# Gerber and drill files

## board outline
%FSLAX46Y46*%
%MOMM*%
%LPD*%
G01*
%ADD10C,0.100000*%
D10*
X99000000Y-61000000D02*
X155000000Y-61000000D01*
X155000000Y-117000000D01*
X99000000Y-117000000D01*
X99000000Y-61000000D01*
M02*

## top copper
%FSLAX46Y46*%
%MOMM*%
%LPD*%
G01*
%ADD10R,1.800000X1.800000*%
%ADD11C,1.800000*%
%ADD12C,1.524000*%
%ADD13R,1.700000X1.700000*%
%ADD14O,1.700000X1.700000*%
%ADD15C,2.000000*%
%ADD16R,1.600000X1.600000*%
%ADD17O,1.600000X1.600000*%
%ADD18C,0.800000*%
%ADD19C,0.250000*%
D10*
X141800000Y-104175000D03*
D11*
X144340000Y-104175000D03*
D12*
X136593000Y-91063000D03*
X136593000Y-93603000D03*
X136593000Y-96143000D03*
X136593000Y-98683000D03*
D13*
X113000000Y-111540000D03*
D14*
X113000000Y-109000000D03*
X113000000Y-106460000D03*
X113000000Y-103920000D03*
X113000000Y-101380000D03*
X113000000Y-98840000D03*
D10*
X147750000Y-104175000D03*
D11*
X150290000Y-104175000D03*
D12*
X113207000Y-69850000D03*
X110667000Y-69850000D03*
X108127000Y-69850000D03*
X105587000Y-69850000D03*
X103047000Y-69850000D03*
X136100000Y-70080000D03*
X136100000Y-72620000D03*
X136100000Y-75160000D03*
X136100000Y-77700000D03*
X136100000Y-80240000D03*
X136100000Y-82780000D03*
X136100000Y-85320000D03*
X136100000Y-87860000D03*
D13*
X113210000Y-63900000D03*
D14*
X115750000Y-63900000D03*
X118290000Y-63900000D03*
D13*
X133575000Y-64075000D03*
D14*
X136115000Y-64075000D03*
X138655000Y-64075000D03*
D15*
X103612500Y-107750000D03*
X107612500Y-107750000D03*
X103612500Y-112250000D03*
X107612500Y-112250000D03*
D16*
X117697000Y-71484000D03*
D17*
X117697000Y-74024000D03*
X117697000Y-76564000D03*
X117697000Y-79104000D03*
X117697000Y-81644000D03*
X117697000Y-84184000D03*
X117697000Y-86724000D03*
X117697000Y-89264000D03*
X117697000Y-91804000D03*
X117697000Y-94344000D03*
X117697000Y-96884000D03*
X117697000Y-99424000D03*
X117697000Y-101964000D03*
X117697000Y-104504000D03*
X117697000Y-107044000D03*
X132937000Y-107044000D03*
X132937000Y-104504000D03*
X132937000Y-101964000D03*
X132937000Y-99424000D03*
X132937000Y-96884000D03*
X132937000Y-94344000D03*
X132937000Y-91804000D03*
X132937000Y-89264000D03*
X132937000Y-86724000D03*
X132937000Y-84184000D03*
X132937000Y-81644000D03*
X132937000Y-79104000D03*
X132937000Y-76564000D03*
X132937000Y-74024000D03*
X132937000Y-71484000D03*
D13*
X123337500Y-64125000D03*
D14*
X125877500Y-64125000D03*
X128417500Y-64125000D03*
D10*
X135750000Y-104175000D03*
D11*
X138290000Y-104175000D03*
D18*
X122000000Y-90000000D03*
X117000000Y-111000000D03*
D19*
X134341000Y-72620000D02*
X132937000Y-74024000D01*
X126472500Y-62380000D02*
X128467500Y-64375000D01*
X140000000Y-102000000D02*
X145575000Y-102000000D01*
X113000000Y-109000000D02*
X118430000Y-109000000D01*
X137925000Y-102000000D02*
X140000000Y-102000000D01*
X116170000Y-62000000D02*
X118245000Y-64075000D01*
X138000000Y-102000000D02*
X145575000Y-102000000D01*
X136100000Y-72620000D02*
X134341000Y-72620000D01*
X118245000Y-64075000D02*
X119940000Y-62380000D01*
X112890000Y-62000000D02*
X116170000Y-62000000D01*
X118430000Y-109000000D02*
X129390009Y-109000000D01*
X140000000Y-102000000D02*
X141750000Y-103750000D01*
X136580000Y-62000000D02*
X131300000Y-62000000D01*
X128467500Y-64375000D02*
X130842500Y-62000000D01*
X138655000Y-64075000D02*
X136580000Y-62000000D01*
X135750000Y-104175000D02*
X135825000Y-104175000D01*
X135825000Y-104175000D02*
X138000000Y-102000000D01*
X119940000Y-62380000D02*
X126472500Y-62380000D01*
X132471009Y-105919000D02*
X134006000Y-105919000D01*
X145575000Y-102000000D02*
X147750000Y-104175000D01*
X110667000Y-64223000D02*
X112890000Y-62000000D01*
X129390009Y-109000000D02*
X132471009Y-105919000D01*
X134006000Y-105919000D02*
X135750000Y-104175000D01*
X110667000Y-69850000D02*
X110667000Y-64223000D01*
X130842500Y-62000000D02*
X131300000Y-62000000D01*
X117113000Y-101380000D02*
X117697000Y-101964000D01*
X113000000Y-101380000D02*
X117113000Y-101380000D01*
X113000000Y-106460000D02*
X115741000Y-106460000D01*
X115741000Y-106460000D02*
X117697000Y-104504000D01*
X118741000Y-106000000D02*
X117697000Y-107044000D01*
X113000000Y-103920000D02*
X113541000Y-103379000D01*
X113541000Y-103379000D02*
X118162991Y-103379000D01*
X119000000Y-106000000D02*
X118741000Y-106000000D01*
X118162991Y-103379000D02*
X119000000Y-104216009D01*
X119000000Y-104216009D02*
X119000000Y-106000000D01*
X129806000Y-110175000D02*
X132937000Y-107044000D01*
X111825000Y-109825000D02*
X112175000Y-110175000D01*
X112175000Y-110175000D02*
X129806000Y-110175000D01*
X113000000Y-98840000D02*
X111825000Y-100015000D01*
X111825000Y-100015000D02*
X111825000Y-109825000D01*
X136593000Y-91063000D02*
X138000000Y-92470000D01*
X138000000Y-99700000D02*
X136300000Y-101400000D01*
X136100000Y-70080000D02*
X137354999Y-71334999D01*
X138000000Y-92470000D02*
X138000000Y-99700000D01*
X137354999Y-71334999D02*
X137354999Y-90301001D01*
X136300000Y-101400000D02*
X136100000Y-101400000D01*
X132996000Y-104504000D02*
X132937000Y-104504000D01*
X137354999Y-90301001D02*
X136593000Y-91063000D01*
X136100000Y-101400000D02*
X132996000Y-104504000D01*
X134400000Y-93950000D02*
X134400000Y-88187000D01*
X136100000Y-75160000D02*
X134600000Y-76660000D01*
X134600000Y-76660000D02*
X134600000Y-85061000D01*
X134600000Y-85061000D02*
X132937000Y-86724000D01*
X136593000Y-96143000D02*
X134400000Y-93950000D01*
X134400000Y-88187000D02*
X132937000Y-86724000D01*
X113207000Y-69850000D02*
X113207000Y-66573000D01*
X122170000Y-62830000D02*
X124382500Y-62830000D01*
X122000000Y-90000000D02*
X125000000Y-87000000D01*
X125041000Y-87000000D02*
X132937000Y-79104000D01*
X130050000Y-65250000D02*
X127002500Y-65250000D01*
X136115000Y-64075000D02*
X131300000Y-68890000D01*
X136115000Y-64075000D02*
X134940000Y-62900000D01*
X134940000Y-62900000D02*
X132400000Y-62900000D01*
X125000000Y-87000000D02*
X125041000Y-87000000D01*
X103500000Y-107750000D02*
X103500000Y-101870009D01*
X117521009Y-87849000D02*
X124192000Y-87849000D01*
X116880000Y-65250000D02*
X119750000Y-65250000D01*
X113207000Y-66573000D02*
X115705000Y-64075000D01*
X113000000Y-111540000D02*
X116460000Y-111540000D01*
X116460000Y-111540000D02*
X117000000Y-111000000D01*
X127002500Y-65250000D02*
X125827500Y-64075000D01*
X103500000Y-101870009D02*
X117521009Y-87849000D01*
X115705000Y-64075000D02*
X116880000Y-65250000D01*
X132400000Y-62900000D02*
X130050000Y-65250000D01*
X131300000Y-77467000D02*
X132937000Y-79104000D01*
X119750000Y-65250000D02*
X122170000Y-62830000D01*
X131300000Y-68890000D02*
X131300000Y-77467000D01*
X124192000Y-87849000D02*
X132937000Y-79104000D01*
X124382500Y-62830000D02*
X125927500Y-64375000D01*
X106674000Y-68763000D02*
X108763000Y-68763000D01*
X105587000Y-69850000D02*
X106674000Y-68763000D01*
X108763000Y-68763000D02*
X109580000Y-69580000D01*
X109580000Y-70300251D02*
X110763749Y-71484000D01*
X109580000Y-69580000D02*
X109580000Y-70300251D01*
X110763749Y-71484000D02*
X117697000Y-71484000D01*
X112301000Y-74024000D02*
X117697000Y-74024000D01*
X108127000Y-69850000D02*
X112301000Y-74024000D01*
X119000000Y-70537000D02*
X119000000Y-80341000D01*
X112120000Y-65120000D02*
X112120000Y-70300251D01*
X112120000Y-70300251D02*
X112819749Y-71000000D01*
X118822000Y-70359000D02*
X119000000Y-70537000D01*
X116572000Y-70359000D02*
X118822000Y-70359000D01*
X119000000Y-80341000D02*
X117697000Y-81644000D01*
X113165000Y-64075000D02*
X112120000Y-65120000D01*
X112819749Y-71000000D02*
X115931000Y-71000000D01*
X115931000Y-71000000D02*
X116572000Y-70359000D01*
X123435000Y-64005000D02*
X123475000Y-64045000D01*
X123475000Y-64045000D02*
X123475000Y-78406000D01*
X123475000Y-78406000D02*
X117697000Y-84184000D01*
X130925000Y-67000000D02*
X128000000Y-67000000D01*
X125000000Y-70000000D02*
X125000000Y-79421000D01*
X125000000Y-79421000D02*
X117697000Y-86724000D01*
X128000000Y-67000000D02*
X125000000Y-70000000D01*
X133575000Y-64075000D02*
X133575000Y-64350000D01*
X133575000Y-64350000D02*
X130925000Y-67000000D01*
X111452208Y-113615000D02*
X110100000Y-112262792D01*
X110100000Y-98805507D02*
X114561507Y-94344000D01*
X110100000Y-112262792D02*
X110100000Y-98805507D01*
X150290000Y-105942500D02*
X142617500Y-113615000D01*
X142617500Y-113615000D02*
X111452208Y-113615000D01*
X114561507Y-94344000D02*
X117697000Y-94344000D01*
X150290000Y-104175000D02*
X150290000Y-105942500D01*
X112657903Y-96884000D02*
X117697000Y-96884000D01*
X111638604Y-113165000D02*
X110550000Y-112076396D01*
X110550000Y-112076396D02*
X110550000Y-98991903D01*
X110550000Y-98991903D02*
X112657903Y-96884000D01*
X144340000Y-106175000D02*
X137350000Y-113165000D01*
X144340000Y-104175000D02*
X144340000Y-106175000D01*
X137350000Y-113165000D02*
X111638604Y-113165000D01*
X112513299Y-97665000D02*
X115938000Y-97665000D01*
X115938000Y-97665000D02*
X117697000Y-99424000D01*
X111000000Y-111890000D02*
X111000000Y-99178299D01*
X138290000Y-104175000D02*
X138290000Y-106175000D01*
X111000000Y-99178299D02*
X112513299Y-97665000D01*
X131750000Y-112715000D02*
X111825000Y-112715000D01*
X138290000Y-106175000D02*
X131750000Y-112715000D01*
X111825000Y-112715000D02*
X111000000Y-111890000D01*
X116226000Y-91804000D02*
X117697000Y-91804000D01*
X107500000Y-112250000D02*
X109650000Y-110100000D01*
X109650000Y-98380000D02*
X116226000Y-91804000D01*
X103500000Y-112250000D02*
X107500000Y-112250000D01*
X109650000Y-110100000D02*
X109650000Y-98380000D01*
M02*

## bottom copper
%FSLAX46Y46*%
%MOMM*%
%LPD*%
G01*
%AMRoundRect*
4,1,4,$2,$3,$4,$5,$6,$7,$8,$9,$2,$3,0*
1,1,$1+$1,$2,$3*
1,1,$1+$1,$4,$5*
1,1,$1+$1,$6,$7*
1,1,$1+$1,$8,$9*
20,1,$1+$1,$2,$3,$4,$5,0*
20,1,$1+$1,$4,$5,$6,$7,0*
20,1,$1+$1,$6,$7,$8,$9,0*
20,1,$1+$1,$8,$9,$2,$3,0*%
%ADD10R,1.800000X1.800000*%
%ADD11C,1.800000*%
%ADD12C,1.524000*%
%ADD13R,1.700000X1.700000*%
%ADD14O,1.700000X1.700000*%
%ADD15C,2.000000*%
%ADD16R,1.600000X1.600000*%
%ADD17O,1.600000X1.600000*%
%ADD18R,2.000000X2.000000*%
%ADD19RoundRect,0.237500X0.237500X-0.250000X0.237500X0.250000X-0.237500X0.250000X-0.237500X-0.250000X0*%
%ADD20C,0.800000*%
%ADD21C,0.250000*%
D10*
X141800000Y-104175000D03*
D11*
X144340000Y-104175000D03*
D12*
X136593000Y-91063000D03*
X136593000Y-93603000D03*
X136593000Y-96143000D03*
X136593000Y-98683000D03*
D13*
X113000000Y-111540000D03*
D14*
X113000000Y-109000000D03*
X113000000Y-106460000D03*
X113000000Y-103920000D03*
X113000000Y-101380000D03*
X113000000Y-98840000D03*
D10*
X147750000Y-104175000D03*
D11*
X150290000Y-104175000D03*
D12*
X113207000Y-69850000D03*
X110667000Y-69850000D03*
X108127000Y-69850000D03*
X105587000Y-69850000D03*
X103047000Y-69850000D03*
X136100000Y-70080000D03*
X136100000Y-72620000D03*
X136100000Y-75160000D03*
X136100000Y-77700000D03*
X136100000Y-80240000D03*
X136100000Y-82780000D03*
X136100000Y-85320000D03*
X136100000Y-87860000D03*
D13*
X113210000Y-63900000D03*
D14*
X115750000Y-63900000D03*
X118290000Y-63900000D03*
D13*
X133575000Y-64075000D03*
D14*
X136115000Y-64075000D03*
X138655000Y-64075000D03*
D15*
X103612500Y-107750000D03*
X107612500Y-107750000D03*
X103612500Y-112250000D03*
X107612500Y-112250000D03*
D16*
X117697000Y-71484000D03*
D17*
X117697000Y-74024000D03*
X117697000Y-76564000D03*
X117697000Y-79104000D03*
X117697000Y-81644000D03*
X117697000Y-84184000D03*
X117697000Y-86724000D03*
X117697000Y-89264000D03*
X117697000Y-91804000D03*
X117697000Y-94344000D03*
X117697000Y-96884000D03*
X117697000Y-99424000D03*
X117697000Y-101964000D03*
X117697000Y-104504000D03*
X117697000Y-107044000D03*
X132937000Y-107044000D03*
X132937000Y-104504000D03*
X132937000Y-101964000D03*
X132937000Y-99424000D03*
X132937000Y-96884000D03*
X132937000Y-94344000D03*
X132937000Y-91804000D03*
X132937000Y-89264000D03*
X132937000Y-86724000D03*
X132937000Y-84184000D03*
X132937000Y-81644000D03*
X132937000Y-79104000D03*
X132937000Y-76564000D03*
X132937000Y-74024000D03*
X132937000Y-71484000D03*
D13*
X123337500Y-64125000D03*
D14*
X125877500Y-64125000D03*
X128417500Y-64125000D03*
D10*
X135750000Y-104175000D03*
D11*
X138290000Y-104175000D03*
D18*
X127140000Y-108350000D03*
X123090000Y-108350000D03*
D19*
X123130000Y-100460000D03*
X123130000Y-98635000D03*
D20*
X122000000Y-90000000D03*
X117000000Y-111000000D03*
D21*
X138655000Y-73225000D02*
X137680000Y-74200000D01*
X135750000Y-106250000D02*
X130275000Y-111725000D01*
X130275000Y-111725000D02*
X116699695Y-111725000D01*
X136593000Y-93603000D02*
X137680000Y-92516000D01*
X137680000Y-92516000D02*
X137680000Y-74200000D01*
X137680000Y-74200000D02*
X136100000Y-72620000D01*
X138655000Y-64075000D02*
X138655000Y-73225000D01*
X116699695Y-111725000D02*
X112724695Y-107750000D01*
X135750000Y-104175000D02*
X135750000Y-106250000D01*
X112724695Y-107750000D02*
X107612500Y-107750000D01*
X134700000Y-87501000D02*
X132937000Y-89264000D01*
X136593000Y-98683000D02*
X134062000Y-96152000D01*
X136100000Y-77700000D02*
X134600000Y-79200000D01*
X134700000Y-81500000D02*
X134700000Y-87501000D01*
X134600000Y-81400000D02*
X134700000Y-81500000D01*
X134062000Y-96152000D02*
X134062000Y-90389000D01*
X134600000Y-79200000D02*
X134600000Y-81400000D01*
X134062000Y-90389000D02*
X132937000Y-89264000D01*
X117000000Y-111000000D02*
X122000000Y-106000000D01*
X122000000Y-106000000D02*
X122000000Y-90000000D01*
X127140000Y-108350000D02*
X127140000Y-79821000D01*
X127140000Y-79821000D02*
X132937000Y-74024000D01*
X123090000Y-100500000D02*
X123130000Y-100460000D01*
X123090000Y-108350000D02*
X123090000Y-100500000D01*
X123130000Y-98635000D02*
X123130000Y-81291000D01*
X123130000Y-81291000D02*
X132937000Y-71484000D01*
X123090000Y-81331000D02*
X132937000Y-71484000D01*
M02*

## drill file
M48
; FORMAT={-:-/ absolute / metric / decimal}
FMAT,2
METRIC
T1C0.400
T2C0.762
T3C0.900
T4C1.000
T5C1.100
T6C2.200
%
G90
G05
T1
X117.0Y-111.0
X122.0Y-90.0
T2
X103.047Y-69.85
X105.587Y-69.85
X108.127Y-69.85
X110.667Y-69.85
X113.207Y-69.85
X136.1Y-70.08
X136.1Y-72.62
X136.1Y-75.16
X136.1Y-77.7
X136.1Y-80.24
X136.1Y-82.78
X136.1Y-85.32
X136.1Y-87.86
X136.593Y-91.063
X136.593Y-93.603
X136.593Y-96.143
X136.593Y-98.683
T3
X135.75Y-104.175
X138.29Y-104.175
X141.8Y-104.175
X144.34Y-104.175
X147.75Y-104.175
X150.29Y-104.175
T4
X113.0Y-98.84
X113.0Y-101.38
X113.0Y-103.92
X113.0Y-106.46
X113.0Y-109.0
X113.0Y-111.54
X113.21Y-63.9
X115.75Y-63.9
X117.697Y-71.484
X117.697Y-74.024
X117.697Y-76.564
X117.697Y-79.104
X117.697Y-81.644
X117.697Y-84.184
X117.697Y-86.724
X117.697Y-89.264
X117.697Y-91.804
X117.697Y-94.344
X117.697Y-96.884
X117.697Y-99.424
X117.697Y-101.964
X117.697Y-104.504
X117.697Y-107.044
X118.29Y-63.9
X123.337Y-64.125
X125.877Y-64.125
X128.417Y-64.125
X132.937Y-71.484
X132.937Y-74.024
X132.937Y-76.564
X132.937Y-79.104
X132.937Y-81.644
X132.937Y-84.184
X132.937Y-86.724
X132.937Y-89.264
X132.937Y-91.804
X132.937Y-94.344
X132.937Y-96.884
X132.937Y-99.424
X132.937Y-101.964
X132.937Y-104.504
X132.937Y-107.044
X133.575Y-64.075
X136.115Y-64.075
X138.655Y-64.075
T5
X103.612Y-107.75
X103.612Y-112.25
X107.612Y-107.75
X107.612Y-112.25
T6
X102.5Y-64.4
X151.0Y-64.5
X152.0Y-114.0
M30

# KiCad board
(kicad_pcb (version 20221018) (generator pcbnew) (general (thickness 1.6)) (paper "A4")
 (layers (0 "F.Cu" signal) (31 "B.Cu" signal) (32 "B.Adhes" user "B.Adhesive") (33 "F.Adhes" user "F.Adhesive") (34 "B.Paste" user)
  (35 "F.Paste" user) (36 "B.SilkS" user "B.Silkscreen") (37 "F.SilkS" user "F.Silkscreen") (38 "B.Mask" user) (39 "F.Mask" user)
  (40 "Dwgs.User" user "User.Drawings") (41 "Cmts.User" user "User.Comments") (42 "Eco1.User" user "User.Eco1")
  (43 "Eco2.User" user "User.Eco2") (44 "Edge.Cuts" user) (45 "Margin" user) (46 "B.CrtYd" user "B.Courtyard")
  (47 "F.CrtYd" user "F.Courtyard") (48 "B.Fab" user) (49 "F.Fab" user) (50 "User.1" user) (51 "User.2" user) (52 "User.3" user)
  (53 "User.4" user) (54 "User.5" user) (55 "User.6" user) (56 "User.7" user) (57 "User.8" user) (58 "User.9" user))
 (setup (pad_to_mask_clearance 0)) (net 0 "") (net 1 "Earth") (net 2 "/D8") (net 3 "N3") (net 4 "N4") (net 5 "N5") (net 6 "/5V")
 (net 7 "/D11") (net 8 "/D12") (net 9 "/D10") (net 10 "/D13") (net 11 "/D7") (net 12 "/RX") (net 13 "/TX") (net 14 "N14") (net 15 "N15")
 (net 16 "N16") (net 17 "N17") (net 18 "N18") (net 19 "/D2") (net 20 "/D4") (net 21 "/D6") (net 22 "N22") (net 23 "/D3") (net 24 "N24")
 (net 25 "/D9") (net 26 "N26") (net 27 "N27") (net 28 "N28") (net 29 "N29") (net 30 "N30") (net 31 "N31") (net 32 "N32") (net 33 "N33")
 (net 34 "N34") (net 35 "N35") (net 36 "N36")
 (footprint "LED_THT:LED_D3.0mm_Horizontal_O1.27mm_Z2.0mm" (layer "F.Cu") (at 141.8 104.175)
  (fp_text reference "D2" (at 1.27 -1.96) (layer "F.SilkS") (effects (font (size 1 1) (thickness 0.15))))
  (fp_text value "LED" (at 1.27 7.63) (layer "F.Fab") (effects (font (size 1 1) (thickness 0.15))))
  (pad "1" thru_hole rect (at 0 0) (size 1.8 1.8) (drill 0.9) (layers "*.Cu" "*.Mask") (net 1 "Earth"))
  (pad "2" thru_hole circle (at 2.54 0) (size 1.8 1.8) (drill 0.9) (layers "*.Cu" "*.Mask") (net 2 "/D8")))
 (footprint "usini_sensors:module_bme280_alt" (layer "F.Cu") (at 136.593 98.683)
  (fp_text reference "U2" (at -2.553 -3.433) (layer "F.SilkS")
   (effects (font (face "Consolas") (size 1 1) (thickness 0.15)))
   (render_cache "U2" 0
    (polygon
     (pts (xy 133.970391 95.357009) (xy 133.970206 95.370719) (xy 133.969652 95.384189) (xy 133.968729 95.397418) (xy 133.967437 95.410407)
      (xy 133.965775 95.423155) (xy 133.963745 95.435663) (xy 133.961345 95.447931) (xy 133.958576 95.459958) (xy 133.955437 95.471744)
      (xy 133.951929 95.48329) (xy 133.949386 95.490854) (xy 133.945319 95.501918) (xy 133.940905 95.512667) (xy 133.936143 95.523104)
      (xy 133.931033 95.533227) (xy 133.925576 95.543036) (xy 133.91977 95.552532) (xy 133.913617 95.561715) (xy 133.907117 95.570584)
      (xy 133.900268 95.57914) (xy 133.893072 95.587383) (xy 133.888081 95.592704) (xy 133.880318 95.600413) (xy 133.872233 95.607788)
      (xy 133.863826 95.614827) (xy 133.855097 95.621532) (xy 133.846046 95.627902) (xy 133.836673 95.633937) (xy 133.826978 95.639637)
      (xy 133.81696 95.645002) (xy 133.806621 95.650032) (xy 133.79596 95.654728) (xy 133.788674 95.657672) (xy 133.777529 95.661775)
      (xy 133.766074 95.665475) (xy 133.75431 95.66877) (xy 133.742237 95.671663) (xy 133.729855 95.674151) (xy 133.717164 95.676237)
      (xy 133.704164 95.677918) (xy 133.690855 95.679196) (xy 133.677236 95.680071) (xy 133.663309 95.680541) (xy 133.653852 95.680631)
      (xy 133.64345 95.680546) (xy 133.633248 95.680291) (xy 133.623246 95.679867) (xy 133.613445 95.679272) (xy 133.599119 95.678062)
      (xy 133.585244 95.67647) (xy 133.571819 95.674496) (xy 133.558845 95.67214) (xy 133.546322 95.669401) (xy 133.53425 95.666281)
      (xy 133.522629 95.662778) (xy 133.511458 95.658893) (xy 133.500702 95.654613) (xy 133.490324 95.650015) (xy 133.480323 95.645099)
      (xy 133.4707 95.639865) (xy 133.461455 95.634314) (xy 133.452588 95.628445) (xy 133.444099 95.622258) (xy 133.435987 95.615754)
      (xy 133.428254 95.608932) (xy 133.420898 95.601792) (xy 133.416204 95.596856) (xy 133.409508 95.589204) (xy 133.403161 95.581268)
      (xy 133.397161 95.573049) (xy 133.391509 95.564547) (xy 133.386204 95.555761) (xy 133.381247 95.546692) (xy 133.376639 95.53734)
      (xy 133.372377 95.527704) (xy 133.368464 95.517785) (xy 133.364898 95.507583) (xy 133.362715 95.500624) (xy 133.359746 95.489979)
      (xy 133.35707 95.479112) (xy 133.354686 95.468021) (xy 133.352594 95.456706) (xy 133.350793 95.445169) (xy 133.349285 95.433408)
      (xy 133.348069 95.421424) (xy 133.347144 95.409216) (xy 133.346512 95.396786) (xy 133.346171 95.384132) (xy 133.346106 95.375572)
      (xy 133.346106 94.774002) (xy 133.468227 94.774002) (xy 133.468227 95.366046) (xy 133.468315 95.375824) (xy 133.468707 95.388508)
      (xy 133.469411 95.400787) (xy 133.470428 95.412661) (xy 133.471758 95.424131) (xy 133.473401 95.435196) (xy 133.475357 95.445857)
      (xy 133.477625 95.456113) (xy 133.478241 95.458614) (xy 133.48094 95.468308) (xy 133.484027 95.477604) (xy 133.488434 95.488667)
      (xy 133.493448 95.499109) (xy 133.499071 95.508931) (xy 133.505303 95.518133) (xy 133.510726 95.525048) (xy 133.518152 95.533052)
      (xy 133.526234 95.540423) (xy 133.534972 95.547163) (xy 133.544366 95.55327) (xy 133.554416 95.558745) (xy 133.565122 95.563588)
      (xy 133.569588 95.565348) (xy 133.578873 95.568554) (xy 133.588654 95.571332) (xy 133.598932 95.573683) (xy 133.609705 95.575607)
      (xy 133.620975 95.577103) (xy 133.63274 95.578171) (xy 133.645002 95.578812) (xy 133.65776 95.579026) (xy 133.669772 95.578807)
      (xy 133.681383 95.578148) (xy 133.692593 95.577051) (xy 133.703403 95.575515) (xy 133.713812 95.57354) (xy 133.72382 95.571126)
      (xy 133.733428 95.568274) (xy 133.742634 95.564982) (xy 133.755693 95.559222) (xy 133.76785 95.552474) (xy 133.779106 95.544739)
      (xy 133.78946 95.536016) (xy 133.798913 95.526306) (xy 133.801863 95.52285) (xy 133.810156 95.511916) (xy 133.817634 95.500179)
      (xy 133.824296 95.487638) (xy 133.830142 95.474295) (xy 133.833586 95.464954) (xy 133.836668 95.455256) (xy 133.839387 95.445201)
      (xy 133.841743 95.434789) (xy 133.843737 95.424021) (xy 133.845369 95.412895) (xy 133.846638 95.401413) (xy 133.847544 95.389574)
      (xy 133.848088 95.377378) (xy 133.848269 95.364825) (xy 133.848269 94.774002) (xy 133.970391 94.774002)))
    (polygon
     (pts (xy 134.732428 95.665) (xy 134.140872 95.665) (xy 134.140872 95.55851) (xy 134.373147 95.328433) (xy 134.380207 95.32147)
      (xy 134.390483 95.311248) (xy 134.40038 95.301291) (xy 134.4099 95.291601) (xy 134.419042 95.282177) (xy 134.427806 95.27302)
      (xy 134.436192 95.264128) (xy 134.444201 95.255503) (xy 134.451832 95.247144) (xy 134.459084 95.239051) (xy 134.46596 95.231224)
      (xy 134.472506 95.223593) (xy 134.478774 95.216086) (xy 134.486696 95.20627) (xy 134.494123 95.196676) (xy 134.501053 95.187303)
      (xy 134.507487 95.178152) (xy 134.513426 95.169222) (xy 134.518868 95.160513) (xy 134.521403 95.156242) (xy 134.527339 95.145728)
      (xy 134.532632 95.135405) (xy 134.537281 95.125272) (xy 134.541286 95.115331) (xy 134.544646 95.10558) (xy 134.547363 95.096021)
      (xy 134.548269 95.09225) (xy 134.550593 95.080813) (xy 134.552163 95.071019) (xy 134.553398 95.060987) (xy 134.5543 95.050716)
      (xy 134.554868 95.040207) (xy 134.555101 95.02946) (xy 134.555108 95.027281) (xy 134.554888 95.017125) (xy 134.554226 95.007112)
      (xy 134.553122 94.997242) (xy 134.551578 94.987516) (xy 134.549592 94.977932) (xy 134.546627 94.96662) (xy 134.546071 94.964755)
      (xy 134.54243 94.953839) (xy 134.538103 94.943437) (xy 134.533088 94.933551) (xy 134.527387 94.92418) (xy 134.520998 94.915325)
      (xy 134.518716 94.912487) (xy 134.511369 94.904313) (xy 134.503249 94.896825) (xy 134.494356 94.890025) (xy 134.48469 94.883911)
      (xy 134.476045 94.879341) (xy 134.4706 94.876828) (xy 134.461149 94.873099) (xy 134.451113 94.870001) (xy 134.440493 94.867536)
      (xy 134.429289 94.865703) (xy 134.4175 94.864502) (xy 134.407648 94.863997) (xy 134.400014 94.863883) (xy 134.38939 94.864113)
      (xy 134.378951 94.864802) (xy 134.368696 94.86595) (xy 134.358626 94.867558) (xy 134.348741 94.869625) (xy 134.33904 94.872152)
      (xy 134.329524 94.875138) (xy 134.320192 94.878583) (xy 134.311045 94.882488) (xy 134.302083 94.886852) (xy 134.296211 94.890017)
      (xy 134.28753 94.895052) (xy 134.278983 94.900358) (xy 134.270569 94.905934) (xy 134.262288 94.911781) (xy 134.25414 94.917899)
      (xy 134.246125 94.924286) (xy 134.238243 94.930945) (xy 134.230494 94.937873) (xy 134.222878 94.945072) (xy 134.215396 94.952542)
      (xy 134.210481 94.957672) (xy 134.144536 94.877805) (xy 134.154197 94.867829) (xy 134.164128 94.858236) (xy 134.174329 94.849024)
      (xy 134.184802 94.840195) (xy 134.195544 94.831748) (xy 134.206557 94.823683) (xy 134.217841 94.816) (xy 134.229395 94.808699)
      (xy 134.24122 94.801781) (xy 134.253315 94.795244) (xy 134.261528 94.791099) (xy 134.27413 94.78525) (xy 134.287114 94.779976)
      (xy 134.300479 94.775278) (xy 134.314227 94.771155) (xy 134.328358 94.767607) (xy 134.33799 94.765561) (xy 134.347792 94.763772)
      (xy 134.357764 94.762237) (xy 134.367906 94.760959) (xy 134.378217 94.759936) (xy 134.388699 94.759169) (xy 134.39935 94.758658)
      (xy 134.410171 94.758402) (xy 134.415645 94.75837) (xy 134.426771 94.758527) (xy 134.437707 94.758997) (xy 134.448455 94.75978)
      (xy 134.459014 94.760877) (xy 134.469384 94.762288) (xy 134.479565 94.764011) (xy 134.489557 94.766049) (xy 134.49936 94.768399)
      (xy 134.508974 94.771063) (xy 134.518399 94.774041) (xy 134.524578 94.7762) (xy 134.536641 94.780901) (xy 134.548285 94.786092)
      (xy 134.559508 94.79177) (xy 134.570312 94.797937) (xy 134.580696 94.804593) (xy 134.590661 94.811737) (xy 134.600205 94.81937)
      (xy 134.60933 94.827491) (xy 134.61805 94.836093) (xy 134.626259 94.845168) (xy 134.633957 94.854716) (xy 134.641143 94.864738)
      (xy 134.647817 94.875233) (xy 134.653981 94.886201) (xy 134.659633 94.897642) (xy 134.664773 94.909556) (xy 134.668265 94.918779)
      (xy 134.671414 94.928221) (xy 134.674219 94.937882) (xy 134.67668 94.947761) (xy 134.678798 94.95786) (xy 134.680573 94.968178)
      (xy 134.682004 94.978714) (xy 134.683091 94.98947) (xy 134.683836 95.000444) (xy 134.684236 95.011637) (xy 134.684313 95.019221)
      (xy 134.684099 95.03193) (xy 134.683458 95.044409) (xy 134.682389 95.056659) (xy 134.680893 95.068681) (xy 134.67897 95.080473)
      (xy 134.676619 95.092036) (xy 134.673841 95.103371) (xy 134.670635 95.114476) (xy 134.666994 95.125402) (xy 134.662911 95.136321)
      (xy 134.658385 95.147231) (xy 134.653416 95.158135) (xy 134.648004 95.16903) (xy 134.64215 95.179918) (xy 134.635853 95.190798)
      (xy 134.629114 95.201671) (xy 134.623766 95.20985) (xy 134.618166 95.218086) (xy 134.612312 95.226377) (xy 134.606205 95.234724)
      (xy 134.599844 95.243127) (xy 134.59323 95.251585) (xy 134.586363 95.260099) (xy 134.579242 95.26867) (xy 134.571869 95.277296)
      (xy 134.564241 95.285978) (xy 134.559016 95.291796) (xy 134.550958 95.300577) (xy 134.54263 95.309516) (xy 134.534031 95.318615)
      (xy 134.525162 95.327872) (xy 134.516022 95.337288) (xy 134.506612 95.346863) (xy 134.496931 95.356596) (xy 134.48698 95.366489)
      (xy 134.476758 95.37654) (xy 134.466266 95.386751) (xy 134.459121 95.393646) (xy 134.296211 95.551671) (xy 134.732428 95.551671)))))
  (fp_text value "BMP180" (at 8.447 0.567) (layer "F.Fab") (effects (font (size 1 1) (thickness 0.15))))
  (pad "1" thru_hole circle (at 0 -7.62) (size 1.524 1.524) (drill 0.762) (layers "*.Cu" "*.Mask") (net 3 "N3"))
  (pad "2" thru_hole circle (at 0 -5.08) (size 1.524 1.524) (drill 0.762) (layers "*.Cu" "*.Mask") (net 1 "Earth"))
  (pad "3" thru_hole circle (at 0 -2.54) (size 1.524 1.524) (drill 0.762) (layers "*.Cu" "*.Mask") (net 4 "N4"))
  (pad "4" thru_hole circle (at 0 0) (size 1.524 1.524) (drill 0.762) (layers "*.Cu" "*.Mask") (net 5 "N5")))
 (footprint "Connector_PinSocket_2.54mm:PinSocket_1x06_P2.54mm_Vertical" (layer "F.Cu") (at 113 111.54 180)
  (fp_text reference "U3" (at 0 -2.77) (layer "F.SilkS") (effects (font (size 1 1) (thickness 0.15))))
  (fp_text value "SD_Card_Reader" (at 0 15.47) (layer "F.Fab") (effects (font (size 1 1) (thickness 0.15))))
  (pad "1" thru_hole rect (at 0 0 180) (size 1.7 1.7) (drill 1) (layers "*.Cu" "*.Mask") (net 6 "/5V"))
  (pad "2" thru_hole oval (at 0 2.54 180) (size 1.7 1.7) (drill 1) (layers "*.Cu" "*.Mask") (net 1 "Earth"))
  (pad "3" thru_hole oval (at 0 5.08 180) (size 1.7 1.7) (drill 1) (layers "*.Cu" "*.Mask") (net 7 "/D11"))
  (pad "4" thru_hole oval (at 0 7.62 180) (size 1.7 1.7) (drill 1) (layers "*.Cu" "*.Mask") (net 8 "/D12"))
  (pad "5" thru_hole oval (at 0 10.16 180) (size 1.7 1.7) (drill 1) (layers "*.Cu" "*.Mask") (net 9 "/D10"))
  (pad "6" thru_hole oval (at 0 12.7 180) (size 1.7 1.7) (drill 1) (layers "*.Cu" "*.Mask") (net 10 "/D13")))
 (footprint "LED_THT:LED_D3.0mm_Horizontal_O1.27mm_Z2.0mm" (layer "F.Cu") (at 147.75 104.175)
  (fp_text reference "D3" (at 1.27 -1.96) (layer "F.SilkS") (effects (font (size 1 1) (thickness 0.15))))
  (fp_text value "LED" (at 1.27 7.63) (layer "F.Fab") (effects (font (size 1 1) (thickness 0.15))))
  (pad "1" thru_hole rect (at 0 0) (size 1.8 1.8) (drill 0.9) (layers "*.Cu" "*.Mask") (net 1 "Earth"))
  (pad "2" thru_hole circle (at 2.54 0) (size 1.8 1.8) (drill 0.9) (layers "*.Cu" "*.Mask") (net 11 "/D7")))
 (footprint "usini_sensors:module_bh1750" (layer "F.Cu") (at 103.047 69.85 -90)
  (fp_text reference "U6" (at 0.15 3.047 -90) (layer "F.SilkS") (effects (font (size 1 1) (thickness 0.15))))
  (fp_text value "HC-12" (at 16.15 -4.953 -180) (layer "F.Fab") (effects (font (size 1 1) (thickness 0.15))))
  (pad "1" thru_hole circle (at 0 -10.16 270) (size 1.524 1.524) (drill 0.762) (layers "*.Cu" "*.Mask") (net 6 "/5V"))
  (pad "2" thru_hole circle (at 0 -7.62 270) (size 1.524 1.524) (drill 0.762) (layers "*.Cu" "*.Mask") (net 1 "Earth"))
  (pad "3" thru_hole circle (at 0 -5.08 270) (size 1.524 1.524) (drill 0.762) (layers "*.Cu" "*.Mask") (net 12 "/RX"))
  (pad "4" thru_hole circle (at 0 -2.54 270) (size 1.524 1.524) (drill 0.762) (layers "*.Cu" "*.Mask") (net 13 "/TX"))
  (pad "5" thru_hole circle (at 0 0 270) (size 1.524 1.524) (drill 0.762) (layers "*.Cu" "*.Mask") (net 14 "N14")))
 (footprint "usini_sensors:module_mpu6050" (layer "F.Cu") (at 136.1 87.86)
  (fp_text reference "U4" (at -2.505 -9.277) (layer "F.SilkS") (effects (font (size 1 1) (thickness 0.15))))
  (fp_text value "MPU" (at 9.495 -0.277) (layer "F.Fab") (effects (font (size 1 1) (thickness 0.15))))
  (pad "1" thru_hole circle (at 0 -17.78) (size 1.524 1.524) (drill 0.762) (layers "*.Cu" "*.Mask") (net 3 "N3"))
  (pad "2" thru_hole circle (at 0 -15.24) (size 1.524 1.524) (drill 0.762) (layers "*.Cu" "*.Mask") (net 1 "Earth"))
  (pad "3" thru_hole circle (at 0 -12.7) (size 1.524 1.524) (drill 0.762) (layers "*.Cu" "*.Mask") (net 4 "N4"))
  (pad "4" thru_hole circle (at 0 -10.16) (size 1.524 1.524) (drill 0.762) (layers "*.Cu" "*.Mask") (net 5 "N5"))
  (pad "5" thru_hole circle (at 0 -7.62) (size 1.524 1.524) (drill 0.762) (layers "*.Cu" "*.Mask") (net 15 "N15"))
  (pad "6" thru_hole circle (at 0 -5.08) (size 1.524 1.524) (drill 0.762) (layers "*.Cu" "*.Mask") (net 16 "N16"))
  (pad "7" thru_hole circle (at 0 -2.54) (size 1.524 1.524) (drill 0.762) (layers "*.Cu" "*.Mask") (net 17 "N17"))
  (pad "8" thru_hole circle (at 0 0) (size 1.524 1.524) (drill 0.762) (layers "*.Cu" "*.Mask") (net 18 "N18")))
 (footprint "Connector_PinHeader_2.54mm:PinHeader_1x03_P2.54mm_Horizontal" (layer "F.Cu") (at 113.16 63.85 90)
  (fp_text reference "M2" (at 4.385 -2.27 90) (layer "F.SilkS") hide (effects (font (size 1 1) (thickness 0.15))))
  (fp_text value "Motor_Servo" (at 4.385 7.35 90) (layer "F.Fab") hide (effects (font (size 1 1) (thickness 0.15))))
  (pad "1" thru_hole rect (at -0.05 0.05 90) (size 1.7 1.7) (drill 1) (layers "*.Cu" "*.Mask") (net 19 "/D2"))
  (pad "2" thru_hole oval (at -0.05 2.59 90) (size 1.7 1.7) (drill 1) (layers "*.Cu" "*.Mask") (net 6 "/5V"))
  (pad "3" thru_hole oval (at -0.05 5.13 90) (size 1.7 1.7) (drill 1) (layers "*.Cu" "*.Mask") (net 1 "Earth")))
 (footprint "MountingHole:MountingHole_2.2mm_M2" (layer "F.Cu") (at 152 114)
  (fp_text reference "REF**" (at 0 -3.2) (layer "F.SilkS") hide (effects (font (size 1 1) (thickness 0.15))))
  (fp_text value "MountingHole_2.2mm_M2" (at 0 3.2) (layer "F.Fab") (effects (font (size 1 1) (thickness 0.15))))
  (pad "" np_thru_hole circle (at 0 0) (size 2.2 2.2) (drill 2.2) (layers "*.Cu" "*.Mask")))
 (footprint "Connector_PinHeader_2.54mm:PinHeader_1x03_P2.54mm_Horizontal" (layer "F.Cu") (at 133.575 64.075 90)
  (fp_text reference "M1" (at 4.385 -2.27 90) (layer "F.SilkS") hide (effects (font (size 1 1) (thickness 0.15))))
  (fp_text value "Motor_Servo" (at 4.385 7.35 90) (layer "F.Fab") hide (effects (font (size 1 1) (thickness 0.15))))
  (pad "1" thru_hole rect (at 0 0 90) (size 1.7 1.7) (drill 1) (layers "*.Cu" "*.Mask") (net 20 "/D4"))
  (pad "2" thru_hole oval (at 0 2.54 90) (size 1.7 1.7) (drill 1) (layers "*.Cu" "*.Mask") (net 6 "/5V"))
  (pad "3" thru_hole oval (at 0 5.08 90) (size 1.7 1.7) (drill 1) (layers "*.Cu" "*.Mask") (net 1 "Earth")))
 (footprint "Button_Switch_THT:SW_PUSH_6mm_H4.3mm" (layer "F.Cu") (at 101.1125 107.75)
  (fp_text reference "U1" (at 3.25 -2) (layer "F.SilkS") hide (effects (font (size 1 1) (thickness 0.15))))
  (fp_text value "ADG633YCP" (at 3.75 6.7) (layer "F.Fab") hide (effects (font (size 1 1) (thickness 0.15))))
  (pad "1" thru_hole circle (at 2.5 0 90) (size 2 2) (drill 1.1) (layers "*.Cu" "*.Mask") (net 6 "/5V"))
  (pad "1" thru_hole circle (at 6.5 0 90) (size 2 2) (drill 1.1) (layers "*.Cu" "*.Mask") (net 1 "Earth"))
  (pad "2" thru_hole circle (at 2.5 4.5 90) (size 2 2) (drill 1.1) (layers "*.Cu" "*.Mask") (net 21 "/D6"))
  (pad "2" thru_hole circle (at 6.5 4.5 90) (size 2 2) (drill 1.1) (layers "*.Cu" "*.Mask") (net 21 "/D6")))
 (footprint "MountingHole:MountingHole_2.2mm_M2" (layer "F.Cu") (at 102.5 64.4)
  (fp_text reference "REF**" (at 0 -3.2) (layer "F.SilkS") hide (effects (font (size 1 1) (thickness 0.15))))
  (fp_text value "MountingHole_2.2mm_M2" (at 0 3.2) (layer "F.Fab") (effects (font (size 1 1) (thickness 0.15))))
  (pad "" np_thru_hole circle (at 0 0) (size 2.2 2.2) (drill 2.2) (layers "*.Cu" "*.Mask")))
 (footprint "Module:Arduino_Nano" (layer "F.Cu") (at 117.697 71.484)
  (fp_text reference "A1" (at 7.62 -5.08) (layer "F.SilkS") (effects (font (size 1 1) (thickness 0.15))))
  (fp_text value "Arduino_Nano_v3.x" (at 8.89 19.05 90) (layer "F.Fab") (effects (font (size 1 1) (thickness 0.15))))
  (pad "1" thru_hole rect (at 0 0) (size 1.6 1.6) (drill 1) (layers "*.Cu" "*.Mask") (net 13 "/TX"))
  (pad "2" thru_hole oval (at 0 2.54) (size 1.6 1.6) (drill 1) (layers "*.Cu" "*.Mask") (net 12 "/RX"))
  (pad "3" thru_hole oval (at 0 5.08) (size 1.6 1.6) (drill 1) (layers "*.Cu" "*.Mask") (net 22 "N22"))
  (pad "4" thru_hole oval (at 0 7.62) (size 1.6 1.6) (drill 1) (layers "*.Cu" "*.Mask") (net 1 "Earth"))
  (pad "5" thru_hole oval (at 0 10.16) (size 1.6 1.6) (drill 1) (layers "*.Cu" "*.Mask") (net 19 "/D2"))
  (pad "6" thru_hole oval (at 0 12.7) (size 1.6 1.6) (drill 1) (layers "*.Cu" "*.Mask") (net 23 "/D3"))
  (pad "7" thru_hole oval (at 0 15.24) (size 1.6 1.6) (drill 1) (layers "*.Cu" "*.Mask") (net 20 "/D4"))
  (pad "8" thru_hole oval (at 0 17.78) (size 1.6 1.6) (drill 1) (layers "*.Cu" "*.Mask") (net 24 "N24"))
  (pad "9" thru_hole oval (at 0 20.32) (size 1.6 1.6) (drill 1) (layers "*.Cu" "*.Mask") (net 21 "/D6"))
  (pad "10" thru_hole oval (at 0 22.86) (size 1.6 1.6) (drill 1) (layers "*.Cu" "*.Mask") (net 11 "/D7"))
  (pad "11" thru_hole oval (at 0 25.4) (size 1.6 1.6) (drill 1) (layers "*.Cu" "*.Mask") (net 2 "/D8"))
  (pad "12" thru_hole oval (at 0 27.94) (size 1.6 1.6) (drill 1) (layers "*.Cu" "*.Mask") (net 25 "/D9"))
  (pad "13" thru_hole oval (at 0 30.48) (size 1.6 1.6) (drill 1) (layers "*.Cu" "*.Mask") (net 9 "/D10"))
  (pad "14" thru_hole oval (at 0 33.02) (size 1.6 1.6) (drill 1) (layers "*.Cu" "*.Mask") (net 7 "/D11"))
  (pad "15" thru_hole oval (at 0 35.56) (size 1.6 1.6) (drill 1) (layers "*.Cu" "*.Mask") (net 8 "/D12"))
  (pad "16" thru_hole oval (at 15.24 35.56) (size 1.6 1.6) (drill 1) (layers "*.Cu" "*.Mask") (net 10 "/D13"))
  (pad "17" thru_hole oval (at 15.24 33.02) (size 1.6 1.6) (drill 1) (layers "*.Cu" "*.Mask") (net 3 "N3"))
  (pad "18" thru_hole oval (at 15.24 30.48) (size 1.6 1.6) (drill 1) (layers "*.Cu" "*.Mask") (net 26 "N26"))
  (pad "19" thru_hole oval (at 15.24 27.94) (size 1.6 1.6) (drill 1) (layers "*.Cu" "*.Mask") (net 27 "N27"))
  (pad "20" thru_hole oval (at 15.24 25.4) (size 1.6 1.6) (drill 1) (layers "*.Cu" "*.Mask") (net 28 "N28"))
  (pad "21" thru_hole oval (at 15.24 22.86) (size 1.6 1.6) (drill 1) (layers "*.Cu" "*.Mask") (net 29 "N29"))
  (pad "22" thru_hole oval (at 15.24 20.32) (size 1.6 1.6) (drill 1) (layers "*.Cu" "*.Mask") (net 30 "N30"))
  (pad "23" thru_hole oval (at 15.24 17.78) (size 1.6 1.6) (drill 1) (layers "*.Cu" "*.Mask") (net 5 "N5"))
  (pad "24" thru_hole oval (at 15.24 15.24) (size 1.6 1.6) (drill 1) (layers "*.Cu" "*.Mask") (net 4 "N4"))
  (pad "25" thru_hole oval (at 15.24 12.7) (size 1.6 1.6) (drill 1) (layers "*.Cu" "*.Mask") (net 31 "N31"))
  (pad "26" thru_hole oval (at 15.24 10.16) (size 1.6 1.6) (drill 1) (layers "*.Cu" "*.Mask") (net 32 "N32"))
  (pad "27" thru_hole oval (at 15.24 7.62) (size 1.6 1.6) (drill 1) (layers "*.Cu" "*.Mask") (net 6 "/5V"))
  (pad "28" thru_hole oval (at 15.24 5.08) (size 1.6 1.6) (drill 1) (layers "*.Cu" "*.Mask") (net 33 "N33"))
  (pad "29" thru_hole oval (at 15.24 2.54) (size 1.6 1.6) (drill 1) (layers "*.Cu" "*.Mask") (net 1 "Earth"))
  (pad "30" thru_hole oval (at 15.24 0) (size 1.6 1.6) (drill 1) (layers "*.Cu" "*.Mask") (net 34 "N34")))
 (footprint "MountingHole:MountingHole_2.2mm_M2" (layer "F.Cu") (at 151 64.5)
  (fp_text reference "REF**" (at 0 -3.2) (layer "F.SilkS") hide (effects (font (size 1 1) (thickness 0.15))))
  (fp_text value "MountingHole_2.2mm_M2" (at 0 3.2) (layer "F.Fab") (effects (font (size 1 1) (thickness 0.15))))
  (pad "" np_thru_hole circle (at 0 0) (size 2.2 2.2) (drill 2.2) (layers "*.Cu" "*.Mask")))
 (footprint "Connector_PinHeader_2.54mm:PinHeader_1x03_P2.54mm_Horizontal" (layer "F.Cu") (at 123.2875 64.075 90)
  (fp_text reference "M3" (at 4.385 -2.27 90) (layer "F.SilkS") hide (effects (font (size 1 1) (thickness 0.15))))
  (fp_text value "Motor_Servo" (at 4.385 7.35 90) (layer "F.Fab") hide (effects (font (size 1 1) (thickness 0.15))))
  (pad "1" thru_hole rect (at -0.05 0.05 90) (size 1.7 1.7) (drill 1) (layers "*.Cu" "*.Mask") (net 23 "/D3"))
  (pad "2" thru_hole oval (at -0.05 2.59 90) (size 1.7 1.7) (drill 1) (layers "*.Cu" "*.Mask") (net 6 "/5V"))
  (pad "3" thru_hole oval (at -0.05 5.13 90) (size 1.7 1.7) (drill 1) (layers "*.Cu" "*.Mask") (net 1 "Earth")))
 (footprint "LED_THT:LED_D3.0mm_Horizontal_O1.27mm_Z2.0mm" (layer "F.Cu") (at 135.75 104.175)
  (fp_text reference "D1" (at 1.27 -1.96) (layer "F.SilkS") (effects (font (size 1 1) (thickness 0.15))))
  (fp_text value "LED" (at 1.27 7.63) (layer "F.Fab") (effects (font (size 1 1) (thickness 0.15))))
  (pad "1" thru_hole rect (at 0 0) (size 1.8 1.8) (drill 0.9) (layers "*.Cu" "*.Mask") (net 1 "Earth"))
  (pad "2" thru_hole circle (at 2.54 0) (size 1.8 1.8) (drill 0.9) (layers "*.Cu" "*.Mask") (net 25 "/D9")))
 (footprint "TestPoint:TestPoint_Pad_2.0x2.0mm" (layer "B.Cu") (at 127.14 108.35 -90)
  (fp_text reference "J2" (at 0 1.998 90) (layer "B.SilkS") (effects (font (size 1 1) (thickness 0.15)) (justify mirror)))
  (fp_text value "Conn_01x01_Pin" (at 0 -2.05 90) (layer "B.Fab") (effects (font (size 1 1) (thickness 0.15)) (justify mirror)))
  (pad "1" smd rect (at 0 0 270) (size 2 2) (layers "B.Cu" "B.Mask") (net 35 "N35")))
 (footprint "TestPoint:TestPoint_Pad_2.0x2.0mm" (layer "B.Cu") (at 123.09 108.35 -90)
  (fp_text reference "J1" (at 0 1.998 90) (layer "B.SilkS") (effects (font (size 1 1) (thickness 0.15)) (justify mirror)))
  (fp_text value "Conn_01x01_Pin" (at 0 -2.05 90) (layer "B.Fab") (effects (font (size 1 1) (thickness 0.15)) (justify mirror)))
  (pad "1" smd rect (at 0 0 270) (size 2 2) (layers "B.Cu" "B.Mask") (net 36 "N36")))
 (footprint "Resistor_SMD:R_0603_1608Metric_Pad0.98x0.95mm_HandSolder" (layer "B.Cu") (at 123.13 99.5475 90)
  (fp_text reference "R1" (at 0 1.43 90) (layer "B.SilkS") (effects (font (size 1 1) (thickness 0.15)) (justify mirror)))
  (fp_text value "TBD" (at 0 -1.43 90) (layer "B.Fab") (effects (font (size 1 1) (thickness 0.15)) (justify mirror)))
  (pad "1" smd roundrect (at -0.9125 0 90) (size 0.975 0.95) (layers "B.Cu" "B.Paste" "B.Mask") (roundrect_rratio 0.25) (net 36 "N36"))
  (pad "2" smd roundrect (at 0.9125 0 90) (size 0.975 0.95) (layers "B.Cu" "B.Paste" "B.Mask") (roundrect_rratio 0.25) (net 34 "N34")))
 (gr_rect (start 99 61) (end 155 117) (stroke (width 0.1) (type default)) (fill none) (layer "Edge.Cuts"))
 (segment (start 134.341 72.62) (end 132.937 74.024) (width 0.25) (layer "F.Cu") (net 1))
 (segment (start 126.4725 62.38) (end 128.4675 64.375) (width 0.25) (layer "F.Cu") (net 1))
 (segment (start 140 102) (end 145.575 102) (width 0.25) (layer "F.Cu") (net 1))
 (segment (start 113 109) (end 118.43 109) (width 0.25) (layer "F.Cu") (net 1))
 (segment (start 137.925 102) (end 140 102) (width 0.25) (layer "F.Cu") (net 1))
 (segment (start 116.17 62) (end 118.245 64.075) (width 0.25) (layer "F.Cu") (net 1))
 (segment (start 138 102) (end 145.575 102) (width 0.25) (layer "F.Cu") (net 1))
 (segment (start 136.1 72.62) (end 134.341 72.62) (width 0.25) (layer "F.Cu") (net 1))
 (segment (start 118.245 64.075) (end 119.94 62.38) (width 0.25) (layer "F.Cu") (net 1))
 (segment (start 112.89 62) (end 116.17 62) (width 0.25) (layer "F.Cu") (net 1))
 (segment (start 118.43 109) (end 129.390009 109) (width 0.25) (layer "F.Cu") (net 1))
 (segment (start 140 102) (end 141.75 103.75) (width 0.25) (layer "F.Cu") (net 1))
 (segment (start 136.58 62) (end 131.3 62) (width 0.25) (layer "F.Cu") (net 1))
 (segment (start 128.4675 64.375) (end 130.8425 62) (width 0.25) (layer "F.Cu") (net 1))
 (segment (start 138.655 64.075) (end 136.58 62) (width 0.25) (layer "F.Cu") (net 1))
 (segment (start 135.75 104.175) (end 135.825 104.175) (width 0.25) (layer "F.Cu") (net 1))
 (segment (start 135.825 104.175) (end 138 102) (width 0.25) (layer "F.Cu") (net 1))
 (segment (start 119.94 62.38) (end 126.4725 62.38) (width 0.25) (layer "F.Cu") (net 1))
 (segment (start 132.471009 105.919) (end 134.006 105.919) (width 0.25) (layer "F.Cu") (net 1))
 (segment (start 145.575 102) (end 147.75 104.175) (width 0.25) (layer "F.Cu") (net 1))
 (segment (start 110.667 64.223) (end 112.89 62) (width 0.25) (layer "F.Cu") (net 1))
 (segment (start 129.390009 109) (end 132.471009 105.919) (width 0.25) (layer "F.Cu") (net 1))
 (segment (start 134.006 105.919) (end 135.75 104.175) (width 0.25) (layer "F.Cu") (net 1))
 (segment (start 110.667 69.85) (end 110.667 64.223) (width 0.25) (layer "F.Cu") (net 1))
 (segment (start 130.8425 62) (end 131.3 62) (width 0.25) (layer "F.Cu") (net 1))
 (segment (start 138.655 73.225) (end 137.68 74.2) (width 0.25) (layer "B.Cu") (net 1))
 (segment (start 135.75 106.25) (end 130.275 111.725) (width 0.25) (layer "B.Cu") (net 1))
 (segment (start 130.275 111.725) (end 116.699695 111.725) (width 0.25) (layer "B.Cu") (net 1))
 (segment (start 136.593 93.603) (end 137.68 92.516) (width 0.25) (layer "B.Cu") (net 1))
 (segment (start 137.68 92.516) (end 137.68 74.2) (width 0.25) (layer "B.Cu") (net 1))
 (segment (start 137.68 74.2) (end 136.1 72.62) (width 0.25) (layer "B.Cu") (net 1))
 (segment (start 138.655 64.075) (end 138.655 73.225) (width 0.25) (layer "B.Cu") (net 1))
 (segment (start 116.699695 111.725) (end 112.724695 107.75) (width 0.25) (layer "B.Cu") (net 1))
 (segment (start 135.75 104.175) (end 135.75 106.25) (width 0.25) (layer "B.Cu") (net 1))
 (segment (start 112.724695 107.75) (end 107.6125 107.75) (width 0.25) (layer "B.Cu") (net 1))
 (segment (start 117.113 101.38) (end 117.697 101.964) (width 0.25) (layer "F.Cu") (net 9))
 (segment (start 113 101.38) (end 117.113 101.38) (width 0.25) (layer "F.Cu") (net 9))
 (segment (start 113 106.46) (end 115.741 106.46) (width 0.25) (layer "F.Cu") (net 7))
 (segment (start 115.741 106.46) (end 117.697 104.504) (width 0.25) (layer "F.Cu") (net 7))
 (segment (start 118.741 106) (end 117.697 107.044) (width 0.25) (layer "F.Cu") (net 8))
 (segment (start 113 103.92) (end 113.541 103.379) (width 0.25) (layer "F.Cu") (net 8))
 (segment (start 113.541 103.379) (end 118.162991 103.379) (width 0.25) (layer "F.Cu") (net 8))
 (segment (start 119 106) (end 118.741 106) (width 0.25) (layer "F.Cu") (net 8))
 (segment (start 118.162991 103.379) (end 119 104.216009) (width 0.25) (layer "F.Cu") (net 8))
 (segment (start 119 104.216009) (end 119 106) (width 0.25) (layer "F.Cu") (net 8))
 (segment (start 129.806 110.175) (end 132.937 107.044) (width 0.25) (layer "F.Cu") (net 10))
 (segment (start 111.825 109.825) (end 112.175 110.175) (width 0.25) (layer "F.Cu") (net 10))
 (segment (start 112.175 110.175) (end 129.806 110.175) (width 0.25) (layer "F.Cu") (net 10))
 (segment (start 113 98.84) (end 111.825 100.015) (width 0.25) (layer "F.Cu") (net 10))
 (segment (start 111.825 100.015) (end 111.825 109.825) (width 0.25) (layer "F.Cu") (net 10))
 (segment (start 136.593 91.063) (end 138 92.47) (width 0.25) (layer "F.Cu") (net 3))
 (segment (start 138 99.7) (end 136.3 101.4) (width 0.25) (layer "F.Cu") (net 3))
 (segment (start 136.1 70.08) (end 137.354999 71.334999) (width 0.25) (layer "F.Cu") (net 3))
 (segment (start 138 92.47) (end 138 99.7) (width 0.25) (layer "F.Cu") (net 3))
 (segment (start 137.354999 71.334999) (end 137.354999 90.301001) (width 0.25) (layer "F.Cu") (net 3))
 (segment (start 136.3 101.4) (end 136.1 101.4) (width 0.25) (layer "F.Cu") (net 3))
 (segment (start 132.996 104.504) (end 132.937 104.504) (width 0.25) (layer "F.Cu") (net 3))
 (segment (start 137.354999 90.301001) (end 136.593 91.063) (width 0.25) (layer "F.Cu") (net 3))
 (segment (start 136.1 101.4) (end 132.996 104.504) (width 0.25) (layer "F.Cu") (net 3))
 (segment (start 134.7 87.501) (end 132.937 89.264) (width 0.25) (layer "B.Cu") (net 5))
 (segment (start 136.593 98.683) (end 134.062 96.152) (width 0.25) (layer "B.Cu") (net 5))
 (segment (start 136.1 77.7) (end 134.6 79.2) (width 0.25) (layer "B.Cu") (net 5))
 (segment (start 134.7 81.5) (end 134.7 87.501) (width 0.25) (layer "B.Cu") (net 5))
 (segment (start 134.6 81.4) (end 134.7 81.5) (width 0.25) (layer "B.Cu") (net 5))
 (segment (start 134.062 96.152) (end 134.062 90.389) (width 0.25) (layer "B.Cu") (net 5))
 (segment (start 134.6 79.2) (end 134.6 81.4) (width 0.25) (layer "B.Cu") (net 5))
 (segment (start 134.062 90.389) (end 132.937 89.264) (width 0.25) (layer "B.Cu") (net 5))
 (segment (start 134.4 93.95) (end 134.4 88.187) (width 0.25) (layer "F.Cu") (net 4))
 (segment (start 136.1 75.16) (end 134.6 76.66) (width 0.25) (layer "F.Cu") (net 4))
 (segment (start 134.6 76.66) (end 134.6 85.061) (width 0.25) (layer "F.Cu") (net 4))
 (segment (start 134.6 85.061) (end 132.937 86.724) (width 0.25) (layer "F.Cu") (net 4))
 (segment (start 136.593 96.143) (end 134.4 93.95) (width 0.25) (layer "F.Cu") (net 4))
 (segment (start 134.4 88.187) (end 132.937 86.724) (width 0.25) (layer "F.Cu") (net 4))
 (segment (start 113.207 69.85) (end 113.207 66.573) (width 0.25) (layer "F.Cu") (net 6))
 (segment (start 122.17 62.83) (end 124.3825 62.83) (width 0.25) (layer "F.Cu") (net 6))
 (segment (start 122 90) (end 125 87) (width 0.25) (layer "F.Cu") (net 6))
 (segment (start 125.041 87) (end 132.937 79.104) (width 0.25) (layer "F.Cu") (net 6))
 (segment (start 130.05 65.25) (end 127.0025 65.25) (width 0.25) (layer "F.Cu") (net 6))
 (segment (start 136.115 64.075) (end 131.3 68.89) (width 0.25) (layer "F.Cu") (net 6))
 (segment (start 136.115 64.075) (end 134.94 62.9) (width 0.25) (layer "F.Cu") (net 6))
 (segment (start 134.94 62.9) (end 132.4 62.9) (width 0.25) (layer "F.Cu") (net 6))
 (segment (start 125 87) (end 125.041 87) (width 0.25) (layer "F.Cu") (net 6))
 (segment (start 103.5 107.75) (end 103.5 101.870009) (width 0.25) (layer "F.Cu") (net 6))
 (segment (start 117.521009 87.849) (end 124.192 87.849) (width 0.25) (layer "F.Cu") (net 6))
 (segment (start 116.88 65.25) (end 119.75 65.25) (width 0.25) (layer "F.Cu") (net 6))
 (segment (start 113.207 66.573) (end 115.705 64.075) (width 0.25) (layer "F.Cu") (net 6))
 (segment (start 113 111.54) (end 116.46 111.54) (width 0.25) (layer "F.Cu") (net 6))
 (segment (start 116.46 111.54) (end 117 111) (width 0.25) (layer "F.Cu") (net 6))
 (segment (start 127.0025 65.25) (end 125.8275 64.075) (width 0.25) (layer "F.Cu") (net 6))
 (segment (start 103.5 101.870009) (end 117.521009 87.849) (width 0.25) (layer "F.Cu") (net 6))
 (segment (start 115.705 64.075) (end 116.88 65.25) (width 0.25) (layer "F.Cu") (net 6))
 (segment (start 132.4 62.9) (end 130.05 65.25) (width 0.25) (layer "F.Cu") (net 6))
 (segment (start 131.3 77.467) (end 132.937 79.104) (width 0.25) (layer "F.Cu") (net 6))
 (segment (start 119.75 65.25) (end 122.17 62.83) (width 0.25) (layer "F.Cu") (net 6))
 (segment (start 131.3 68.89) (end 131.3 77.467) (width 0.25) (layer "F.Cu") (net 6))
 (segment (start 124.192 87.849) (end 132.937 79.104) (width 0.25) (layer "F.Cu") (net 6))
 (segment (start 124.3825 62.83) (end 125.9275 64.375) (width 0.25) (layer "F.Cu") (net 6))
 (via (at 122 90) (size 0.8) (drill 0.4) (layers "F.Cu" "B.Cu") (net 6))
 (via (at 117 111) (size 0.8) (drill 0.4) (layers "F.Cu" "B.Cu") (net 6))
 (segment (start 117 111) (end 122 106) (width 0.25) (layer "B.Cu") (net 6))
 (segment (start 122 106) (end 122 90) (width 0.25) (layer "B.Cu") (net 6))
 (segment (start 106.674 68.763) (end 108.763 68.763) (width 0.25) (layer "F.Cu") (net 13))
 (segment (start 105.587 69.85) (end 106.674 68.763) (width 0.25) (layer "F.Cu") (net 13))
 (segment (start 108.763 68.763) (end 109.58 69.58) (width 0.25) (layer "F.Cu") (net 13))
 (segment (start 109.58 70.300251) (end 110.763749 71.484) (width 0.25) (layer "F.Cu") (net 13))
 (segment (start 109.58 69.58) (end 109.58 70.300251) (width 0.25) (layer "F.Cu") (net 13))
 (segment (start 110.763749 71.484) (end 117.697 71.484) (width 0.25) (layer "F.Cu") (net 13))
 (segment (start 112.301 74.024) (end 117.697 74.024) (width 0.25) (layer "F.Cu") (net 12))
 (segment (start 108.127 69.85) (end 112.301 74.024) (width 0.25) (layer "F.Cu") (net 12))
 (segment (start 119 70.537) (end 119 80.341) (width 0.25) (layer "F.Cu") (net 19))
 (segment (start 112.12 65.12) (end 112.12 70.300251) (width 0.25) (layer "F.Cu") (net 19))
 (segment (start 112.12 70.300251) (end 112.819749 71) (width 0.25) (layer "F.Cu") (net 19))
 (segment (start 118.822 70.359) (end 119 70.537) (width 0.25) (layer "F.Cu") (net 19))
 (segment (start 116.572 70.359) (end 118.822 70.359) (width 0.25) (layer "F.Cu") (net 19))
 (segment (start 119 80.341) (end 117.697 81.644) (width 0.25) (layer "F.Cu") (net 19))
 (segment (start 113.165 64.075) (end 112.12 65.12) (width 0.25) (layer "F.Cu") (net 19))
 (segment (start 112.819749 71) (end 115.931 71) (width 0.25) (layer "F.Cu") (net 19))
 (segment (start 115.931 71) (end 116.572 70.359) (width 0.25) (layer "F.Cu") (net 19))
 (segment (start 123.435 64.005) (end 123.475 64.045) (width 0.25) (layer "F.Cu") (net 23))
 (segment (start 123.475 64.045) (end 123.475 78.406) (width 0.25) (layer "F.Cu") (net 23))
 (segment (start 123.475 78.406) (end 117.697 84.184) (width 0.25) (layer "F.Cu") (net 23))
 (segment (start 130.925 67) (end 128 67) (width 0.25) (layer "F.Cu") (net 20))
 (segment (start 125 70) (end 125 79.421) (width 0.25) (layer "F.Cu") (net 20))
 (segment (start 125 79.421) (end 117.697 86.724) (width 0.25) (layer "F.Cu") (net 20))
 (segment (start 128 67) (end 125 70) (width 0.25) (layer "F.Cu") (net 20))
 (segment (start 133.575 64.075) (end 133.575 64.35) (width 0.25) (layer "F.Cu") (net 20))
 (segment (start 133.575 64.35) (end 130.925 67) (width 0.25) (layer "F.Cu") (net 20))
 (segment (start 111.452208 113.615) (end 110.1 112.262792) (width 0.25) (layer "F.Cu") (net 11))
 (segment (start 110.1 98.805507) (end 114.561507 94.344) (width 0.25) (layer "F.Cu") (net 11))
 (segment (start 110.1 112.262792) (end 110.1 98.805507) (width 0.25) (layer "F.Cu") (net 11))
 (segment (start 150.29 105.9425) (end 142.6175 113.615) (width 0.25) (layer "F.Cu") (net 11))
 (segment (start 142.6175 113.615) (end 111.452208 113.615) (width 0.25) (layer "F.Cu") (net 11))
 (segment (start 114.561507 94.344) (end 117.697 94.344) (width 0.25) (layer "F.Cu") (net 11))
 (segment (start 150.29 104.175) (end 150.29 105.9425) (width 0.25) (layer "F.Cu") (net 11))
 (segment (start 112.657903 96.884) (end 117.697 96.884) (width 0.25) (layer "F.Cu") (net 2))
 (segment (start 111.638604 113.165) (end 110.55 112.076396) (width 0.25) (layer "F.Cu") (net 2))
 (segment (start 110.55 112.076396) (end 110.55 98.991903) (width 0.25) (layer "F.Cu") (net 2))
 (segment (start 110.55 98.991903) (end 112.657903 96.884) (width 0.25) (layer "F.Cu") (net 2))
 (segment (start 144.34 106.175) (end 137.35 113.165) (width 0.25) (layer "F.Cu") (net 2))
 (segment (start 144.34 104.175) (end 144.34 106.175) (width 0.25) (layer "F.Cu") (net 2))
 (segment (start 137.35 113.165) (end 111.638604 113.165) (width 0.25) (layer "F.Cu") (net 2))
 (segment (start 112.513299 97.665) (end 115.938 97.665) (width 0.25) (layer "F.Cu") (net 25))
 (segment (start 115.938 97.665) (end 117.697 99.424) (width 0.25) (layer "F.Cu") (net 25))
 (segment (start 111 111.89) (end 111 99.178299) (width 0.25) (layer "F.Cu") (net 25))
 (segment (start 138.29 104.175) (end 138.29 106.175) (width 0.25) (layer "F.Cu") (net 25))
 (segment (start 111 99.178299) (end 112.513299 97.665) (width 0.25) (layer "F.Cu") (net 25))
 (segment (start 131.75 112.715) (end 111.825 112.715) (width 0.25) (layer "F.Cu") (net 25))
 (segment (start 138.29 106.175) (end 131.75 112.715) (width 0.25) (layer "F.Cu") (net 25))
 (segment (start 111.825 112.715) (end 111 111.89) (width 0.25) (layer "F.Cu") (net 25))
 (segment (start 116.226 91.804) (end 117.697 91.804) (width 0.25) (layer "F.Cu") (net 21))
 (segment (start 107.5 112.25) (end 109.65 110.1) (width 0.25) (layer "F.Cu") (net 21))
 (segment (start 109.65 98.38) (end 116.226 91.804) (width 0.25) (layer "F.Cu") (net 21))
 (segment (start 103.5 112.25) (end 107.5 112.25) (width 0.25) (layer "F.Cu") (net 21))
 (segment (start 109.65 110.1) (end 109.65 98.38) (width 0.25) (layer "F.Cu") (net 21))
 (segment (start 127.14 108.35) (end 127.14 79.821) (width 0.25) (layer "B.Cu") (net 35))
 (segment (start 127.14 79.821) (end 132.937 74.024) (width 0.25) (layer "B.Cu") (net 35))
 (segment (start 123.09 100.5) (end 123.13 100.46) (width 0.25) (layer "B.Cu") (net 36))
 (segment (start 123.09 108.35) (end 123.09 100.5) (width 0.25) (layer "B.Cu") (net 36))
 (segment (start 123.13 98.635) (end 123.13 81.291) (width 0.25) (layer "B.Cu") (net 34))
 (segment (start 123.13 81.291) (end 132.937 71.484) (width 0.25) (layer "B.Cu") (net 34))
 (segment (start 123.09 81.331) (end 132.937 71.484) (width 0.25) (layer "B.Cu") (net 34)))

